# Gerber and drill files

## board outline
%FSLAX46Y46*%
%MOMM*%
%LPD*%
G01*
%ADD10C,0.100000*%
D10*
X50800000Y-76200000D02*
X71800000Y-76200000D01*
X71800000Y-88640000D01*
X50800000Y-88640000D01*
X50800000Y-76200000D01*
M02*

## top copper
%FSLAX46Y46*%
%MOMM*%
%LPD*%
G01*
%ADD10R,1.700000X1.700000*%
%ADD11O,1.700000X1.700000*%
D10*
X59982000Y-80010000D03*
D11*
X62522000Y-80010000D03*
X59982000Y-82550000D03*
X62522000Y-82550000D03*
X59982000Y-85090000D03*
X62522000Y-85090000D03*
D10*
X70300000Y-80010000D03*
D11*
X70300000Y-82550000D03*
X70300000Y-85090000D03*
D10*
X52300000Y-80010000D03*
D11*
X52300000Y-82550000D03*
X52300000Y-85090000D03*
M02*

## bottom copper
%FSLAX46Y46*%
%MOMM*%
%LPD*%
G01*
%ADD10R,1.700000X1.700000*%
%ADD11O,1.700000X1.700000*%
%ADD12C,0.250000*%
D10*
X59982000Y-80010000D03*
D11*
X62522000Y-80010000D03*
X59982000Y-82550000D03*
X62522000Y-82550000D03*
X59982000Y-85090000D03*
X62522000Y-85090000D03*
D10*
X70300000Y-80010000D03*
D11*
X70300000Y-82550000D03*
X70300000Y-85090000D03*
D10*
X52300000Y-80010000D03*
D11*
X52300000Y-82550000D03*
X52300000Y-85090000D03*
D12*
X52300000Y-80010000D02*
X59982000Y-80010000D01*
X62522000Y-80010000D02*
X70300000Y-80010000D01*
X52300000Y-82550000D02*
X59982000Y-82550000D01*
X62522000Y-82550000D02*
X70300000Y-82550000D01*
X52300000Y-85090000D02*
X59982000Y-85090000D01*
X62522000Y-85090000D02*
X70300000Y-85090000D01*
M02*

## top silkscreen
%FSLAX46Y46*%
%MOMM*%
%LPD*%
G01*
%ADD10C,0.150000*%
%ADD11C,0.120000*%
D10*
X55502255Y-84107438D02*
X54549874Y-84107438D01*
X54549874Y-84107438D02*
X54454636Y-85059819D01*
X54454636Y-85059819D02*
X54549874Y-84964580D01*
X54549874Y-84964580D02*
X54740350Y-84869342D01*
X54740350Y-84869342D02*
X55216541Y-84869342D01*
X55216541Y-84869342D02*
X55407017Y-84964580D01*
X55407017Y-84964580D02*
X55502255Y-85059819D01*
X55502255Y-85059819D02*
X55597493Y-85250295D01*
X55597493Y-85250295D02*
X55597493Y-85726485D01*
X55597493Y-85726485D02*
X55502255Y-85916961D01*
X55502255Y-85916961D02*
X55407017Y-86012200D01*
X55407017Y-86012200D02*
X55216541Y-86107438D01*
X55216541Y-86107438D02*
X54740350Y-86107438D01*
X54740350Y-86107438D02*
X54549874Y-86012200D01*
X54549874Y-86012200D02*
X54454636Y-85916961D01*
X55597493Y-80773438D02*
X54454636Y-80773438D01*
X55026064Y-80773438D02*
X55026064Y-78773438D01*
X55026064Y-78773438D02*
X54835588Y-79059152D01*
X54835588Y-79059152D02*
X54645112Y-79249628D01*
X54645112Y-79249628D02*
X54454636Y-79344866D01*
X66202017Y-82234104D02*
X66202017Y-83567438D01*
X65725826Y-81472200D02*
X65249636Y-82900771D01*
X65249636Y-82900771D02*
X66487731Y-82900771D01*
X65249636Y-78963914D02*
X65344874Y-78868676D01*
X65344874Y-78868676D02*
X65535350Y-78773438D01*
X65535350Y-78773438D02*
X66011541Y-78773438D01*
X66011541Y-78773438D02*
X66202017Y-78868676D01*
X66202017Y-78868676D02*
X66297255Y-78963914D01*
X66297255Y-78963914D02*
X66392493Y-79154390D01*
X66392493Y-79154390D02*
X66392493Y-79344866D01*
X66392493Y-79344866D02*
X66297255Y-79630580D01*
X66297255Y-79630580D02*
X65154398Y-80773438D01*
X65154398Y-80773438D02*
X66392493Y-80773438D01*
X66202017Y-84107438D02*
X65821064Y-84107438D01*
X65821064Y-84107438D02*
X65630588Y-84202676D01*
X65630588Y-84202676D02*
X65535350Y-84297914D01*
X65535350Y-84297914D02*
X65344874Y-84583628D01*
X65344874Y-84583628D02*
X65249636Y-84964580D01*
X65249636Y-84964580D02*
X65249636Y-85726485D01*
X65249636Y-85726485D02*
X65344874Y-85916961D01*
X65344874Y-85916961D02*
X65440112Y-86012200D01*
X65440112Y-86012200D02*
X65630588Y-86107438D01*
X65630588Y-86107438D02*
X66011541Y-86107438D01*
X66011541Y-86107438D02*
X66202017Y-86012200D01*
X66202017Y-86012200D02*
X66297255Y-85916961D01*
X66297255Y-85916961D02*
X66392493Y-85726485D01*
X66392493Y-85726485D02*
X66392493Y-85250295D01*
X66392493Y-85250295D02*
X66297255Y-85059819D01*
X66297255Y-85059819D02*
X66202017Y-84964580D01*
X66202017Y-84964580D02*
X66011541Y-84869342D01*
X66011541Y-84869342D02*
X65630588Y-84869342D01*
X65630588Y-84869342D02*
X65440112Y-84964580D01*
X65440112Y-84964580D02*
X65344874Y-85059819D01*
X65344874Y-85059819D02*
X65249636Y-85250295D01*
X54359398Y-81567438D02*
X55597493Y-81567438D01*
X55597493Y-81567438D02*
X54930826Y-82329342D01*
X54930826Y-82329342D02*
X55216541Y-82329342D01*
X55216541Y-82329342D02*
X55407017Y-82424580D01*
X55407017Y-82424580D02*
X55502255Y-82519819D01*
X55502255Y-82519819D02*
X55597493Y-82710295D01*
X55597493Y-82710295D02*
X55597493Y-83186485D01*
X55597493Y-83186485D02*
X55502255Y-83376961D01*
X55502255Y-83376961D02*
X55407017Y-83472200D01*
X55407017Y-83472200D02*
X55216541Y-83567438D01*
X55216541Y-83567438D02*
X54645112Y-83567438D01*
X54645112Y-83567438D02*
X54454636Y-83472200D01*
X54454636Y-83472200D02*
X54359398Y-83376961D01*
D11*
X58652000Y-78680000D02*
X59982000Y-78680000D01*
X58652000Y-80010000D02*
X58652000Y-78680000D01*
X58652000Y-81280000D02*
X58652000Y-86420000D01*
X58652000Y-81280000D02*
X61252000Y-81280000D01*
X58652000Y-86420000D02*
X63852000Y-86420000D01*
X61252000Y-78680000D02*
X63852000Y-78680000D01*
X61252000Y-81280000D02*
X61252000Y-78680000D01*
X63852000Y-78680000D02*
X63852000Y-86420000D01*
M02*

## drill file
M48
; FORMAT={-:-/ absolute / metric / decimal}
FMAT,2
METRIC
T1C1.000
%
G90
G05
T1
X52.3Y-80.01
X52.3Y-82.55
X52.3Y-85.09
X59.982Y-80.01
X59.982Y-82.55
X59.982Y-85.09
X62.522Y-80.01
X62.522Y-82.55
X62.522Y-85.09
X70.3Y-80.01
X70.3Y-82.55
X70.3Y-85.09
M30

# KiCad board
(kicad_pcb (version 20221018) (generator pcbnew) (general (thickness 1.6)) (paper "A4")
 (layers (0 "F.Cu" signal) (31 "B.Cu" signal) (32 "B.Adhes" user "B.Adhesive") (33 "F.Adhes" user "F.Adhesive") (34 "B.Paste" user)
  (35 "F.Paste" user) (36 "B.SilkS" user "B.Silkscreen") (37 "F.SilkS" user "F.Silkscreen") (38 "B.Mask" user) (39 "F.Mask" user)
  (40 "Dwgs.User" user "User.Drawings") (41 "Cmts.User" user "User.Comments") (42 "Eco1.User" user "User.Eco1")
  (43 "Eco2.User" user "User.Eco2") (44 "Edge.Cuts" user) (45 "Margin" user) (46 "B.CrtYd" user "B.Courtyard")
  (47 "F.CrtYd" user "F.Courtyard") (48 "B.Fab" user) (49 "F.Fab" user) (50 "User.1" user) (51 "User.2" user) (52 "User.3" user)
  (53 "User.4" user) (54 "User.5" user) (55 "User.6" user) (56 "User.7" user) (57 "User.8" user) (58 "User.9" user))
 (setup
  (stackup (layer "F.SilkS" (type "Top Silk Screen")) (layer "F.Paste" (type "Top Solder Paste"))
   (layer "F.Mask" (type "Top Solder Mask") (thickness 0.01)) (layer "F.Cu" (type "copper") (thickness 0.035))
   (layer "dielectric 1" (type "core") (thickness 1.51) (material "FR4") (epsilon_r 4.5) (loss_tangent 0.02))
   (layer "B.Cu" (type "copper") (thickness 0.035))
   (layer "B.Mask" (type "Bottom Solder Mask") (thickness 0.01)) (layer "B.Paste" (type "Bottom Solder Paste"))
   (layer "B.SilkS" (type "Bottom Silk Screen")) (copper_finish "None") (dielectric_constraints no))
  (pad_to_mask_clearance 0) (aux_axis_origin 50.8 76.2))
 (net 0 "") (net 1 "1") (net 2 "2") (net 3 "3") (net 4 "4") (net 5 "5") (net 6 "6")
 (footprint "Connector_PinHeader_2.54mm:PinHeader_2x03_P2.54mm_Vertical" (layer "F.Cu") (at 59.982 80.01)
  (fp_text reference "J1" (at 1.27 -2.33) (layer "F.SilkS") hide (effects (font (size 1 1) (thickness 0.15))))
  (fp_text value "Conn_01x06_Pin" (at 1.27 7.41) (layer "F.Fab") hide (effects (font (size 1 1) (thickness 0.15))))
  (fp_line (start -1.33 -1.33) (end 0 -1.33) (stroke (width 0.12) (type solid)) (layer "F.SilkS"))
  (fp_line (start -1.33 0) (end -1.33 -1.33) (stroke (width 0.12) (type solid)) (layer "F.SilkS"))
  (fp_line (start -1.33 1.27) (end -1.33 6.41) (stroke (width 0.12) (type solid)) (layer "F.SilkS"))
  (fp_line (start -1.33 1.27) (end 1.27 1.27) (stroke (width 0.12) (type solid)) (layer "F.SilkS"))
  (fp_line (start -1.33 6.41) (end 3.87 6.41) (stroke (width 0.12) (type solid)) (layer "F.SilkS"))
  (fp_line (start 1.27 -1.33) (end 3.87 -1.33) (stroke (width 0.12) (type solid)) (layer "F.SilkS"))
  (fp_line (start 1.27 1.27) (end 1.27 -1.33) (stroke (width 0.12) (type solid)) (layer "F.SilkS"))
  (fp_line (start 3.87 -1.33) (end 3.87 6.41) (stroke (width 0.12) (type solid)) (layer "F.SilkS"))
  (pad "1" thru_hole rect (at 0 0) (size 1.7 1.7) (drill 1) (layers "*.Cu" "*.Mask") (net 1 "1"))
  (pad "2" thru_hole oval (at 2.54 0) (size 1.7 1.7) (drill 1) (layers "*.Cu" "*.Mask") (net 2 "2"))
  (pad "3" thru_hole oval (at 0 2.54) (size 1.7 1.7) (drill 1) (layers "*.Cu" "*.Mask") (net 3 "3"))
  (pad "4" thru_hole oval (at 2.54 2.54) (size 1.7 1.7) (drill 1) (layers "*.Cu" "*.Mask") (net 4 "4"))
  (pad "5" thru_hole oval (at 0 5.08) (size 1.7 1.7) (drill 1) (layers "*.Cu" "*.Mask") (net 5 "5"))
  (pad "6" thru_hole oval (at 2.54 5.08) (size 1.7 1.7) (drill 1) (layers "*.Cu" "*.Mask") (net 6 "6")))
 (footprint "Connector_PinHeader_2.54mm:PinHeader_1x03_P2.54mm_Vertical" (layer "B.Cu") (at 70.3 80.01 180)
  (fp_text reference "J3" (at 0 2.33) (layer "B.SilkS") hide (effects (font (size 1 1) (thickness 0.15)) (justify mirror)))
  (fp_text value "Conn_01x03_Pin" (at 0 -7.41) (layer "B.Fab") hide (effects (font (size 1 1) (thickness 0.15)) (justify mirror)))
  (pad "1" thru_hole rect (at 0 0 180) (size 1.7 1.7) (drill 1) (layers "*.Cu" "*.Mask") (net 2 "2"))
  (pad "2" thru_hole oval (at 0 -2.54 180) (size 1.7 1.7) (drill 1) (layers "*.Cu" "*.Mask") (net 4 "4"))
  (pad "3" thru_hole oval (at 0 -5.08 180) (size 1.7 1.7) (drill 1) (layers "*.Cu" "*.Mask") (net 6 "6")))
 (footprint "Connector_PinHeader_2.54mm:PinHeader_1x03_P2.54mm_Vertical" (layer "B.Cu") (at 52.3 80.01 180)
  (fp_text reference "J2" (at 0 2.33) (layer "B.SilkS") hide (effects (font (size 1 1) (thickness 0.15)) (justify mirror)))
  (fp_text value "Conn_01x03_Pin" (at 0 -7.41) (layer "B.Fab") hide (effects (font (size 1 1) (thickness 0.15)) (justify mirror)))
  (pad "1" thru_hole rect (at 0 0 180) (size 1.7 1.7) (drill 1) (layers "*.Cu" "*.Mask") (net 1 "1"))
  (pad "2" thru_hole oval (at 0 -2.54 180) (size 1.7 1.7) (drill 1) (layers "*.Cu" "*.Mask") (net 3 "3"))
  (pad "3" thru_hole oval (at 0 -5.08 180) (size 1.7 1.7) (drill 1) (layers "*.Cu" "*.Mask") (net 5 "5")))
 (gr_rect (start 50.8 76.2) (end 71.8 88.64) (stroke (width 0.1) (type default)) (fill none) (layer "Edge.Cuts"))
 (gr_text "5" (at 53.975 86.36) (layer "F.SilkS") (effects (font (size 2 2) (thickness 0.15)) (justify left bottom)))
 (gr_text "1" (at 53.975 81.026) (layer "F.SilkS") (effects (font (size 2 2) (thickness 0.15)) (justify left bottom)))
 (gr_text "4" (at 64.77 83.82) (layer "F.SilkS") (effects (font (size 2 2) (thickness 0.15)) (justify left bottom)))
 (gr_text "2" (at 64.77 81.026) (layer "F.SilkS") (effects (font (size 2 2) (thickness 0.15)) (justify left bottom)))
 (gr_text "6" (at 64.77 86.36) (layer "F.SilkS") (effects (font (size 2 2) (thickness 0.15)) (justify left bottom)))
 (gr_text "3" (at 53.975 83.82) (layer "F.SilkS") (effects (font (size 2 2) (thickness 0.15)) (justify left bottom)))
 (segment (start 52.3 80.01) (end 59.982 80.01) (width 0.25) (layer "B.Cu") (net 1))
 (segment (start 62.522 80.01) (end 70.3 80.01) (width 0.25) (layer "B.Cu") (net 2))
 (segment (start 52.3 82.55) (end 59.982 82.55) (width 0.25) (layer "B.Cu") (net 3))
 (segment (start 62.522 82.55) (end 70.3 82.55) (width 0.25) (layer "B.Cu") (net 4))
 (segment (start 52.3 85.09) (end 59.982 85.09) (width 0.25) (layer "B.Cu") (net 5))
 (segment (start 62.522 85.09) (end 70.3 85.09) (width 0.25) (layer "B.Cu") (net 6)))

